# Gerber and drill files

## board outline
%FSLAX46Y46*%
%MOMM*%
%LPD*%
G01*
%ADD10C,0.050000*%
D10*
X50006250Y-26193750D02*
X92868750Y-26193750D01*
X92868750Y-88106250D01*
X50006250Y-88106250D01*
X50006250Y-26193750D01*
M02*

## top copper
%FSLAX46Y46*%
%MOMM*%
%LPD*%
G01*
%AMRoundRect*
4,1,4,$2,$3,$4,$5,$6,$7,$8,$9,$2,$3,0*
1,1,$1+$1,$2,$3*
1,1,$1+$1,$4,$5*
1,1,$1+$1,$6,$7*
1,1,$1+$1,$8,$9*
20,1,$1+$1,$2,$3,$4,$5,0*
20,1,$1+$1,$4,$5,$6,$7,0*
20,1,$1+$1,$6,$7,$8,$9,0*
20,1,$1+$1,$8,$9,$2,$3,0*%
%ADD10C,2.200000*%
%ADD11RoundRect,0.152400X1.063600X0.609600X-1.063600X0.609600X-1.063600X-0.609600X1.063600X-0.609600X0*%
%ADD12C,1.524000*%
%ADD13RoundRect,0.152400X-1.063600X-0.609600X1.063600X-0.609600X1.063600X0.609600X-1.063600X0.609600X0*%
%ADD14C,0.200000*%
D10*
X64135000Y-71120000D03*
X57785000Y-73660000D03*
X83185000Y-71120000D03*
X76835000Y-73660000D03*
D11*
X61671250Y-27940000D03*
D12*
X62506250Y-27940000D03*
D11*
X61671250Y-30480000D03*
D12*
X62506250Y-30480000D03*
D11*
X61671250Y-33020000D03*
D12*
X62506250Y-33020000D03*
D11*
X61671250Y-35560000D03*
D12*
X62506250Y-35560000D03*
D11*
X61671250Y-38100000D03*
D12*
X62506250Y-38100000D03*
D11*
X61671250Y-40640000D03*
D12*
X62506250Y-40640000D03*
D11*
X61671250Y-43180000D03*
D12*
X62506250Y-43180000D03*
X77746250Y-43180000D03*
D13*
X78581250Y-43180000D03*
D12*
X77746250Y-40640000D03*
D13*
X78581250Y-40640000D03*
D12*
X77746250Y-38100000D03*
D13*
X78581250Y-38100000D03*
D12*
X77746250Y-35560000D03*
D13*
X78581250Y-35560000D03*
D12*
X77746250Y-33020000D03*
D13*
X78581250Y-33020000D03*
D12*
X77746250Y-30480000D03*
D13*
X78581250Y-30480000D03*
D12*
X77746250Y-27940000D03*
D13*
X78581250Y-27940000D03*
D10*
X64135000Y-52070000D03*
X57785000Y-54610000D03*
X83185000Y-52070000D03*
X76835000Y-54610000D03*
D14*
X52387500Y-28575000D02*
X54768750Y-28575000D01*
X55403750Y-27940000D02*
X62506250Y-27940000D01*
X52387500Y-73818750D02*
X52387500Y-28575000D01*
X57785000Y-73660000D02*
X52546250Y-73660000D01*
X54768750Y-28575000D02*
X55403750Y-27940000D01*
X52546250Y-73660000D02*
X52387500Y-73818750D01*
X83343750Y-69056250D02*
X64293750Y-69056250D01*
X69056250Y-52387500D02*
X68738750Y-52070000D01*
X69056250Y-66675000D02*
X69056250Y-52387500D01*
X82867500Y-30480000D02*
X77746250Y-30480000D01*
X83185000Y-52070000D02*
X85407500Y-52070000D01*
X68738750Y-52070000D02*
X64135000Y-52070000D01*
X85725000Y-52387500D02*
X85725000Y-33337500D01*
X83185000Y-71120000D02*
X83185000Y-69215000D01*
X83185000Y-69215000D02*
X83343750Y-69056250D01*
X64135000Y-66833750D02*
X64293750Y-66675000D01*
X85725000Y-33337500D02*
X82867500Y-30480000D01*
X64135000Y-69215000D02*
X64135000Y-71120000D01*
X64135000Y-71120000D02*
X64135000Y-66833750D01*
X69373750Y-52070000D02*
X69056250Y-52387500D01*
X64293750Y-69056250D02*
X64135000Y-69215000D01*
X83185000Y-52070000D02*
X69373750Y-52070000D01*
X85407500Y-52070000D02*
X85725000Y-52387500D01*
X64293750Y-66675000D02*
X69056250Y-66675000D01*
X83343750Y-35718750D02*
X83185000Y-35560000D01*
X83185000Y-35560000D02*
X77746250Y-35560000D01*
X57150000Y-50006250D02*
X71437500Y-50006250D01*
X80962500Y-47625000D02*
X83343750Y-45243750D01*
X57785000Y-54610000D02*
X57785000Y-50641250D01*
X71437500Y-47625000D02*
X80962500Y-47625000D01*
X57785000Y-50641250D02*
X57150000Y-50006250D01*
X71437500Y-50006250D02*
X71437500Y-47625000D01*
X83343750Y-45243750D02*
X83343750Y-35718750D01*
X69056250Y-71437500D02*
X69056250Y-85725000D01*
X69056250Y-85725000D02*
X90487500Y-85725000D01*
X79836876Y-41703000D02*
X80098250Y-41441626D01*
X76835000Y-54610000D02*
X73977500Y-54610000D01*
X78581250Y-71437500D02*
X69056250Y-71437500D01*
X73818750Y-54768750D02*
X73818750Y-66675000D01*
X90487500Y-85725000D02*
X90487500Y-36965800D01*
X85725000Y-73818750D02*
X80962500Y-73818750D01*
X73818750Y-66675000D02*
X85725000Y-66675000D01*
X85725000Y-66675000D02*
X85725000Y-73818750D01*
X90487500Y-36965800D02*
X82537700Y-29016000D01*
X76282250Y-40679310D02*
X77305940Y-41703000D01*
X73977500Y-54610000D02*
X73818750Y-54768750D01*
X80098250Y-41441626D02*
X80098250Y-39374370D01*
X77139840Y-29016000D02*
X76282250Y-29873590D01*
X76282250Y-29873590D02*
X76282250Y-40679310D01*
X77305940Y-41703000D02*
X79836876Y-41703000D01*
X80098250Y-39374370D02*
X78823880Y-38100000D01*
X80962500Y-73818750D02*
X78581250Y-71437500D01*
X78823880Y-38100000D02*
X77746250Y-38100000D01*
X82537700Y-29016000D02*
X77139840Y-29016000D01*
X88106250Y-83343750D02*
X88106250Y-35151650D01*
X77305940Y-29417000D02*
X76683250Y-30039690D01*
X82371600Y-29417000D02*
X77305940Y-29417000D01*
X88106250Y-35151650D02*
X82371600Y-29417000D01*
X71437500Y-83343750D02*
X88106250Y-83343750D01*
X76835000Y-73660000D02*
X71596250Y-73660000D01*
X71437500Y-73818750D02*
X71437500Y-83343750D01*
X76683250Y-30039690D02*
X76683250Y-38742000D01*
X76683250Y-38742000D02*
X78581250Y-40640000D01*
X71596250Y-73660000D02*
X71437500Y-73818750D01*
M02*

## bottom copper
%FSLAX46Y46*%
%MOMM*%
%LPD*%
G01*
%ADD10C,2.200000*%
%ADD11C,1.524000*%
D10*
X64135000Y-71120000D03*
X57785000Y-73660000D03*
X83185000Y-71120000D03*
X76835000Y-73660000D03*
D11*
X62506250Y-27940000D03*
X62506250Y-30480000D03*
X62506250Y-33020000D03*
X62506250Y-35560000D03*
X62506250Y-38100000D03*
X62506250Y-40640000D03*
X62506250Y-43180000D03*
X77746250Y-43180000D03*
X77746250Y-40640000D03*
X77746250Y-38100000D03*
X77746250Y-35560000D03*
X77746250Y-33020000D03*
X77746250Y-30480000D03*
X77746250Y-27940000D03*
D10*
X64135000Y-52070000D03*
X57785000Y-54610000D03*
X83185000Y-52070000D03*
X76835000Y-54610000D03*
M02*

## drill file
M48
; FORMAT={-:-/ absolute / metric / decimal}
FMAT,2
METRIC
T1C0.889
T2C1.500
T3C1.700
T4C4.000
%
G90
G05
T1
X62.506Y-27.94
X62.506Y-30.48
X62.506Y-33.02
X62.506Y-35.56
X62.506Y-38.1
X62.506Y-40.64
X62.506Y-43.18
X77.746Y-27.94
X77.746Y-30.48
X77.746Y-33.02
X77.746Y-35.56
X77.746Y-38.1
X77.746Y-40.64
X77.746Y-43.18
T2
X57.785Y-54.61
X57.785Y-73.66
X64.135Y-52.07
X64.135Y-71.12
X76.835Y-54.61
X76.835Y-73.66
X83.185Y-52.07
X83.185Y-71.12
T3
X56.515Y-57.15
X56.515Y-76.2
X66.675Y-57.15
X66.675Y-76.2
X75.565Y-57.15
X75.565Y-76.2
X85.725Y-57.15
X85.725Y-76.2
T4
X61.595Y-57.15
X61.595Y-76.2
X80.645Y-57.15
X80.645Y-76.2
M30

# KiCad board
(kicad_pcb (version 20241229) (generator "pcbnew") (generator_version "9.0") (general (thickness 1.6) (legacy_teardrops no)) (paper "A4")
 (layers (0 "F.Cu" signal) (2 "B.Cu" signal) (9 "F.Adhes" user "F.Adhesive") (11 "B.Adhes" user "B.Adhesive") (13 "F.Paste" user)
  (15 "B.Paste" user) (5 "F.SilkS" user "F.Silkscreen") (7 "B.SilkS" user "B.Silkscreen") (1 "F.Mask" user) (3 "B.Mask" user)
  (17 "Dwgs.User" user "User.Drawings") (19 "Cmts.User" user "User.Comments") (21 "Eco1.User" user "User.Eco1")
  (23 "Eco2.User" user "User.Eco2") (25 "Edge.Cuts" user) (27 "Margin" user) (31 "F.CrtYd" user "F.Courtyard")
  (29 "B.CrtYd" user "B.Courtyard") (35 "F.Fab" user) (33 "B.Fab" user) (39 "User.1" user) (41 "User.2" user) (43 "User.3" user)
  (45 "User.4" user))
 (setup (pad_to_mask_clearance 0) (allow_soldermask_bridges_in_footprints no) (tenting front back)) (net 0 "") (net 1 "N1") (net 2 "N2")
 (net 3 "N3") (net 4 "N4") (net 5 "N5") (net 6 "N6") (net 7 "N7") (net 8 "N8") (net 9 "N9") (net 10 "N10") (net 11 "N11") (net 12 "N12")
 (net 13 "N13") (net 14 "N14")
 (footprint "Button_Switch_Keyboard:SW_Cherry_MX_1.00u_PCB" (layer "F.Cu") (at 64.135 71.12)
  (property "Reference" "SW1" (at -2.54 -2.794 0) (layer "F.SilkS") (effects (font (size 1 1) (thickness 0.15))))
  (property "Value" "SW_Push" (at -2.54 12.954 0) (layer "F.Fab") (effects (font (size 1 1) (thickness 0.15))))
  (pad "" np_thru_hole circle (at -7.62 5.08) (size 1.7 1.7) (drill 1.7) (layers "*.Cu" "*.Mask"))
  (pad "" np_thru_hole circle (at -2.54 5.08) (size 4 4) (drill 4) (layers "*.Cu" "*.Mask"))
  (pad "" np_thru_hole circle (at 2.54 5.08) (size 1.7 1.7) (drill 1.7) (layers "*.Cu" "*.Mask"))
  (pad "1" thru_hole circle (at 0 0) (size 2.2 2.2) (drill 1.5) (layers "*.Cu" "*.Mask") (remove_unused_layers no) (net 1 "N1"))
  (pad "2" thru_hole circle (at -6.35 2.54) (size 2.2 2.2) (drill 1.5) (layers "*.Cu" "*.Mask") (remove_unused_layers no) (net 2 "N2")))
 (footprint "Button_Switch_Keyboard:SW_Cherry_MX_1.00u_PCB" (layer "F.Cu") (at 83.185 71.12)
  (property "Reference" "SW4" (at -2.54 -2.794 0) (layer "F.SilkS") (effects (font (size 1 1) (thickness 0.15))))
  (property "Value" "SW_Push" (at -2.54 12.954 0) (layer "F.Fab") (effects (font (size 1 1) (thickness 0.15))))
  (pad "" np_thru_hole circle (at -7.62 5.08) (size 1.7 1.7) (drill 1.7) (layers "*.Cu" "*.Mask"))
  (pad "" np_thru_hole circle (at -2.54 5.08) (size 4 4) (drill 4) (layers "*.Cu" "*.Mask"))
  (pad "" np_thru_hole circle (at 2.54 5.08) (size 1.7 1.7) (drill 1.7) (layers "*.Cu" "*.Mask"))
  (pad "1" thru_hole circle (at 0 0) (size 2.2 2.2) (drill 1.5) (layers "*.Cu" "*.Mask") (remove_unused_layers no) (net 1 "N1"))
  (pad "2" thru_hole circle (at -6.35 2.54) (size 2.2 2.2) (drill 1.5) (layers "*.Cu" "*.Mask") (remove_unused_layers no) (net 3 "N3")))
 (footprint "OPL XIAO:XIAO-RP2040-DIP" (layer "F.Cu") (at 70.12625 35.56)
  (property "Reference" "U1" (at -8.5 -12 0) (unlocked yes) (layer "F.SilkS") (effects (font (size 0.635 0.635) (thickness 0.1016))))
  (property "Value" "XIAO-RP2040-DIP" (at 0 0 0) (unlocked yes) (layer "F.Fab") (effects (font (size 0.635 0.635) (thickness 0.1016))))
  (pad "1" smd roundrect (at -8.455 -7.62 180) (size 2.432 1.524) (layers "F.Cu" "F.Mask") (roundrect_rratio 0.1) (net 2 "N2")
   (thermal_bridge_angle 45))
  (pad "1" thru_hole circle (at -7.62 -7.62 180) (size 1.524 1.524) (drill 0.889) (layers "*.Cu" "*.Mask") (remove_unused_layers no)
   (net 2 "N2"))
  (pad "2" smd roundrect (at -8.455 -5.08 180) (size 2.432 1.524) (layers "F.Cu" "F.Mask") (roundrect_rratio 0.1) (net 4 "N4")
   (thermal_bridge_angle 45))
  (pad "2" thru_hole circle (at -7.62 -5.08 180) (size 1.524 1.524) (drill 0.889) (layers "*.Cu" "*.Mask") (remove_unused_layers no)
   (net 4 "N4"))
  (pad "3" smd roundrect (at -8.455 -2.54 180) (size 2.432 1.524) (layers "F.Cu" "F.Mask") (roundrect_rratio 0.1) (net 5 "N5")
   (thermal_bridge_angle 45))
  (pad "3" thru_hole circle (at -7.62 -2.54 180) (size 1.524 1.524) (drill 0.889) (layers "*.Cu" "*.Mask") (remove_unused_layers no)
   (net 5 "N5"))
  (pad "4" smd roundrect (at -8.455 0 180) (size 2.432 1.524) (layers "F.Cu" "F.Mask") (roundrect_rratio 0.1) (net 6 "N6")
   (thermal_bridge_angle 45))
  (pad "4" thru_hole circle (at -7.62 0 180) (size 1.524 1.524) (drill 0.889) (layers "*.Cu" "*.Mask") (remove_unused_layers no)
   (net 6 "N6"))
  (pad "5" smd roundrect (at -8.455 2.54 180) (size 2.432 1.524) (layers "F.Cu" "F.Mask") (roundrect_rratio 0.1) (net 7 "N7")
   (thermal_bridge_angle 45))
  (pad "5" thru_hole circle (at -7.62 2.54 180) (size 1.524 1.524) (drill 0.889) (layers "*.Cu" "*.Mask") (remove_unused_layers no)
   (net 7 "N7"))
  (pad "6" smd roundrect (at -8.455 5.08 180) (size 2.432 1.524) (layers "F.Cu" "F.Mask") (roundrect_rratio 0.1) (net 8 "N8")
   (thermal_bridge_angle 45))
  (pad "6" thru_hole circle (at -7.62 5.08 180) (size 1.524 1.524) (drill 0.889) (layers "*.Cu" "*.Mask") (remove_unused_layers no)
   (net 8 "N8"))
  (pad "7" smd roundrect (at -8.455 7.62 180) (size 2.432 1.524) (layers "F.Cu" "F.Mask") (roundrect_rratio 0.1) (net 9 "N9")
   (thermal_bridge_angle 45))
  (pad "7" thru_hole circle (at -7.62 7.62 180) (size 1.524 1.524) (drill 0.889) (layers "*.Cu" "*.Mask") (remove_unused_layers no)
   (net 9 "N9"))
  (pad "8" thru_hole circle (at 7.62 7.62) (size 1.524 1.524) (drill 0.889) (layers "*.Cu" "*.Mask") (remove_unused_layers no)
   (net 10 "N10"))
  (pad "8" smd roundrect (at 8.455 7.62) (size 2.432 1.524) (layers "F.Cu" "F.Mask") (roundrect_rratio 0.1) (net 10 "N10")
   (thermal_bridge_angle 45))
  (pad "9" thru_hole circle (at 7.62 5.08) (size 1.524 1.524) (drill 0.889) (layers "*.Cu" "*.Mask") (remove_unused_layers no) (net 3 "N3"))
  (pad "9" smd roundrect (at 8.455 5.08) (size 2.432 1.524) (layers "F.Cu" "F.Mask") (roundrect_rratio 0.1) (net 3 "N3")
   (thermal_bridge_angle 45))
  (pad "10" thru_hole circle (at 7.62 2.54) (size 1.524 1.524) (drill 0.889) (layers "*.Cu" "*.Mask") (remove_unused_layers no)
   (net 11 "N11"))
  (pad "10" smd roundrect (at 8.455 2.54) (size 2.432 1.524) (layers "F.Cu" "F.Mask") (roundrect_rratio 0.1) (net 11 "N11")
   (thermal_bridge_angle 45))
  (pad "11" thru_hole circle (at 7.62 0) (size 1.524 1.524) (drill 0.889) (layers "*.Cu" "*.Mask") (remove_unused_layers no) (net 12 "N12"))
  (pad "11" smd roundrect (at 8.455 0) (size 2.432 1.524) (layers "F.Cu" "F.Mask") (roundrect_rratio 0.1) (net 12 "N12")
   (thermal_bridge_angle 45))
  (pad "12" thru_hole circle (at 7.62 -2.54) (size 1.524 1.524) (drill 0.889) (layers "*.Cu" "*.Mask") (remove_unused_layers no)
   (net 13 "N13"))
  (pad "12" smd roundrect (at 8.455 -2.54) (size 2.432 1.524) (layers "F.Cu" "F.Mask") (roundrect_rratio 0.1) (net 13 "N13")
   (thermal_bridge_angle 45))
  (pad "13" thru_hole circle (at 7.62 -5.08) (size 1.524 1.524) (drill 0.889) (layers "*.Cu" "*.Mask") (remove_unused_layers no)
   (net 1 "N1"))
  (pad "13" smd roundrect (at 8.455 -5.08) (size 2.432 1.524) (layers "F.Cu" "F.Mask") (roundrect_rratio 0.1) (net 1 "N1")
   (thermal_bridge_angle 45))
  (pad "14" thru_hole circle (at 7.62 -7.62) (size 1.524 1.524) (drill 0.889) (layers "*.Cu" "*.Mask") (remove_unused_layers no)
   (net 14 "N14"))
  (pad "14" smd roundrect (at 8.455 -7.62) (size 2.432 1.524) (layers "F.Cu" "F.Mask") (roundrect_rratio 0.1) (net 14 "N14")
   (thermal_bridge_angle 45)))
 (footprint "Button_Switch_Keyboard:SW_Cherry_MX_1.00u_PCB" (layer "F.Cu") (at 64.135 52.07)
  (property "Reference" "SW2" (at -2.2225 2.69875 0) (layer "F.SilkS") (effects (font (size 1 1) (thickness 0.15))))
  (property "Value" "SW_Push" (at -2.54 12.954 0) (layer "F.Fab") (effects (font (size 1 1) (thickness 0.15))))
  (pad "" np_thru_hole circle (at -7.62 5.08) (size 1.7 1.7) (drill 1.7) (layers "*.Cu" "*.Mask"))
  (pad "" np_thru_hole circle (at -2.54 5.08) (size 4 4) (drill 4) (layers "*.Cu" "*.Mask"))
  (pad "" np_thru_hole circle (at 2.54 5.08) (size 1.7 1.7) (drill 1.7) (layers "*.Cu" "*.Mask"))
  (pad "1" thru_hole circle (at 0 0) (size 2.2 2.2) (drill 1.5) (layers "*.Cu" "*.Mask") (remove_unused_layers no) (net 1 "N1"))
  (pad "2" thru_hole circle (at -6.35 2.54) (size 2.2 2.2) (drill 1.5) (layers "*.Cu" "*.Mask") (remove_unused_layers no) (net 12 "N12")))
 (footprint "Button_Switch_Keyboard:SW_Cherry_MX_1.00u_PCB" (layer "F.Cu") (at 83.185 52.07)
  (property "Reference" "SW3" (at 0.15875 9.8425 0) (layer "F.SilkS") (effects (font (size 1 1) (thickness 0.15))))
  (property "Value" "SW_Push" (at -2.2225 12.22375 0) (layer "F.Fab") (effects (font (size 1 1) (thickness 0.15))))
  (pad "" np_thru_hole circle (at -7.62 5.08) (size 1.7 1.7) (drill 1.7) (layers "*.Cu" "*.Mask"))
  (pad "" np_thru_hole circle (at -2.54 5.08) (size 4 4) (drill 4) (layers "*.Cu" "*.Mask"))
  (pad "" np_thru_hole circle (at 2.54 5.08) (size 1.7 1.7) (drill 1.7) (layers "*.Cu" "*.Mask"))
  (pad "1" thru_hole circle (at 0 0) (size 2.2 2.2) (drill 1.5) (layers "*.Cu" "*.Mask") (remove_unused_layers no) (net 1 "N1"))
  (pad "2" thru_hole circle (at -6.35 2.54) (size 2.2 2.2) (drill 1.5) (layers "*.Cu" "*.Mask") (remove_unused_layers no) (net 11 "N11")))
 (gr_rect (start 50.00625 26.19375) (end 92.86875 88.10625) (stroke (width 0.05) (type default)) (fill no) (layer "Edge.Cuts"))
 (segment (start 52.3875 28.575) (end 54.76875 28.575) (width 0.2) (layer "F.Cu") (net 2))
 (segment (start 55.40375 27.94) (end 62.50625 27.94) (width 0.2) (layer "F.Cu") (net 2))
 (segment (start 52.3875 73.81875) (end 52.3875 28.575) (width 0.2) (layer "F.Cu") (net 2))
 (segment (start 57.785 73.66) (end 52.54625 73.66) (width 0.2) (layer "F.Cu") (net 2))
 (segment (start 54.76875 28.575) (end 55.40375 27.94) (width 0.2) (layer "F.Cu") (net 2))
 (segment (start 52.54625 73.66) (end 52.3875 73.81875) (width 0.2) (layer "F.Cu") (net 2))
 (segment (start 83.34375 69.05625) (end 64.29375 69.05625) (width 0.2) (layer "F.Cu") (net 1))
 (segment (start 69.05625 52.3875) (end 68.73875 52.07) (width 0.2) (layer "F.Cu") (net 1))
 (segment (start 69.05625 66.675) (end 69.05625 52.3875) (width 0.2) (layer "F.Cu") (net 1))
 (segment (start 82.8675 30.48) (end 77.74625 30.48) (width 0.2) (layer "F.Cu") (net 1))
 (segment (start 83.185 52.07) (end 85.4075 52.07) (width 0.2) (layer "F.Cu") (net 1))
 (segment (start 68.73875 52.07) (end 64.135 52.07) (width 0.2) (layer "F.Cu") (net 1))
 (segment (start 85.725 52.3875) (end 85.725 33.3375) (width 0.2) (layer "F.Cu") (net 1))
 (segment (start 83.185 71.12) (end 83.185 69.215) (width 0.2) (layer "F.Cu") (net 1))
 (segment (start 83.185 69.215) (end 83.34375 69.05625) (width 0.2) (layer "F.Cu") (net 1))
 (segment (start 64.135 66.83375) (end 64.29375 66.675) (width 0.2) (layer "F.Cu") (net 1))
 (segment (start 85.725 33.3375) (end 82.8675 30.48) (width 0.2) (layer "F.Cu") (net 1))
 (segment (start 64.135 69.215) (end 64.135 71.12) (width 0.2) (layer "F.Cu") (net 1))
 (segment (start 64.135 71.12) (end 64.135 66.83375) (width 0.2) (layer "F.Cu") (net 1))
 (segment (start 69.37375 52.07) (end 69.05625 52.3875) (width 0.2) (layer "F.Cu") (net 1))
 (segment (start 64.29375 69.05625) (end 64.135 69.215) (width 0.2) (layer "F.Cu") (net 1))
 (segment (start 83.185 52.07) (end 69.37375 52.07) (width 0.2) (layer "F.Cu") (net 1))
 (segment (start 85.4075 52.07) (end 85.725 52.3875) (width 0.2) (layer "F.Cu") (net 1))
 (segment (start 64.29375 66.675) (end 69.05625 66.675) (width 0.2) (layer "F.Cu") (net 1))
 (segment (start 83.34375 35.71875) (end 83.185 35.56) (width 0.2) (layer "F.Cu") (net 12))
 (segment (start 83.185 35.56) (end 77.74625 35.56) (width 0.2) (layer "F.Cu") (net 12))
 (segment (start 57.15 50.00625) (end 71.4375 50.00625) (width 0.2) (layer "F.Cu") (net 12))
 (segment (start 80.9625 47.625) (end 83.34375 45.24375) (width 0.2) (layer "F.Cu") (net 12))
 (segment (start 57.785 54.61) (end 57.785 50.64125) (width 0.2) (layer "F.Cu") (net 12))
 (segment (start 71.4375 47.625) (end 80.9625 47.625) (width 0.2) (layer "F.Cu") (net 12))
 (segment (start 57.785 50.64125) (end 57.15 50.00625) (width 0.2) (layer "F.Cu") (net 12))
 (segment (start 71.4375 50.00625) (end 71.4375 47.625) (width 0.2) (layer "F.Cu") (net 12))
 (segment (start 83.34375 45.24375) (end 83.34375 35.71875) (width 0.2) (layer "F.Cu") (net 12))
 (segment (start 69.05625 71.4375) (end 69.05625 85.725) (width 0.2) (layer "F.Cu") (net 11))
 (segment (start 69.05625 85.725) (end 90.4875 85.725) (width 0.2) (layer "F.Cu") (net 11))
 (segment (start 79.836876 41.703) (end 80.09825 41.441626) (width 0.2) (layer "F.Cu") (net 11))
 (segment (start 76.835 54.61) (end 73.9775 54.61) (width 0.2) (layer "F.Cu") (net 11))
 (segment (start 78.58125 71.4375) (end 69.05625 71.4375) (width 0.2) (layer "F.Cu") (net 11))
 (segment (start 73.81875 54.76875) (end 73.81875 66.675) (width 0.2) (layer "F.Cu") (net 11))
 (segment (start 90.4875 85.725) (end 90.4875 36.9658) (width 0.2) (layer "F.Cu") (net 11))
 (segment (start 85.725 73.81875) (end 80.9625 73.81875) (width 0.2) (layer "F.Cu") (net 11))
 (segment (start 73.81875 66.675) (end 85.725 66.675) (width 0.2) (layer "F.Cu") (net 11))
 (segment (start 85.725 66.675) (end 85.725 73.81875) (width 0.2) (layer "F.Cu") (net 11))
 (segment (start 90.4875 36.9658) (end 82.5377 29.016) (width 0.2) (layer "F.Cu") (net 11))
 (segment (start 76.28225 40.67931) (end 77.30594 41.703) (width 0.2) (layer "F.Cu") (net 11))
 (segment (start 73.9775 54.61) (end 73.81875 54.76875) (width 0.2) (layer "F.Cu") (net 11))
 (segment (start 80.09825 41.441626) (end 80.09825 39.37437) (width 0.2) (layer "F.Cu") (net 11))
 (segment (start 77.13984 29.016) (end 76.28225 29.87359) (width 0.2) (layer "F.Cu") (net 11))
 (segment (start 76.28225 29.87359) (end 76.28225 40.67931) (width 0.2) (layer "F.Cu") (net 11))
 (segment (start 77.30594 41.703) (end 79.836876 41.703) (width 0.2) (layer "F.Cu") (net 11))
 (segment (start 80.09825 39.37437) (end 78.82388 38.1) (width 0.2) (layer "F.Cu") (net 11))
 (segment (start 80.9625 73.81875) (end 78.58125 71.4375) (width 0.2) (layer "F.Cu") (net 11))
 (segment (start 78.82388 38.1) (end 77.74625 38.1) (width 0.2) (layer "F.Cu") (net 11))
 (segment (start 82.5377 29.016) (end 77.13984 29.016) (width 0.2) (layer "F.Cu") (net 11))
 (segment (start 88.10625 83.34375) (end 88.10625 35.15165) (width 0.2) (layer "F.Cu") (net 3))
 (segment (start 77.30594 29.417) (end 76.68325 30.03969) (width 0.2) (layer "F.Cu") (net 3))
 (segment (start 82.3716 29.417) (end 77.30594 29.417) (width 0.2) (layer "F.Cu") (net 3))
 (segment (start 88.10625 35.15165) (end 82.3716 29.417) (width 0.2) (layer "F.Cu") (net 3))
 (segment (start 71.4375 83.34375) (end 88.10625 83.34375) (width 0.2) (layer "F.Cu") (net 3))
 (segment (start 76.835 73.66) (end 71.59625 73.66) (width 0.2) (layer "F.Cu") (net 3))
 (segment (start 71.4375 73.81875) (end 71.4375 83.34375) (width 0.2) (layer "F.Cu") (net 3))
 (segment (start 76.68325 30.03969) (end 76.68325 38.742) (width 0.2) (layer "F.Cu") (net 3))
 (segment (start 76.68325 38.742) (end 78.58125 40.64) (width 0.2) (layer "F.Cu") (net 3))
 (segment (start 71.59625 73.66) (end 71.4375 73.81875) (width 0.2) (layer "F.Cu") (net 3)))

